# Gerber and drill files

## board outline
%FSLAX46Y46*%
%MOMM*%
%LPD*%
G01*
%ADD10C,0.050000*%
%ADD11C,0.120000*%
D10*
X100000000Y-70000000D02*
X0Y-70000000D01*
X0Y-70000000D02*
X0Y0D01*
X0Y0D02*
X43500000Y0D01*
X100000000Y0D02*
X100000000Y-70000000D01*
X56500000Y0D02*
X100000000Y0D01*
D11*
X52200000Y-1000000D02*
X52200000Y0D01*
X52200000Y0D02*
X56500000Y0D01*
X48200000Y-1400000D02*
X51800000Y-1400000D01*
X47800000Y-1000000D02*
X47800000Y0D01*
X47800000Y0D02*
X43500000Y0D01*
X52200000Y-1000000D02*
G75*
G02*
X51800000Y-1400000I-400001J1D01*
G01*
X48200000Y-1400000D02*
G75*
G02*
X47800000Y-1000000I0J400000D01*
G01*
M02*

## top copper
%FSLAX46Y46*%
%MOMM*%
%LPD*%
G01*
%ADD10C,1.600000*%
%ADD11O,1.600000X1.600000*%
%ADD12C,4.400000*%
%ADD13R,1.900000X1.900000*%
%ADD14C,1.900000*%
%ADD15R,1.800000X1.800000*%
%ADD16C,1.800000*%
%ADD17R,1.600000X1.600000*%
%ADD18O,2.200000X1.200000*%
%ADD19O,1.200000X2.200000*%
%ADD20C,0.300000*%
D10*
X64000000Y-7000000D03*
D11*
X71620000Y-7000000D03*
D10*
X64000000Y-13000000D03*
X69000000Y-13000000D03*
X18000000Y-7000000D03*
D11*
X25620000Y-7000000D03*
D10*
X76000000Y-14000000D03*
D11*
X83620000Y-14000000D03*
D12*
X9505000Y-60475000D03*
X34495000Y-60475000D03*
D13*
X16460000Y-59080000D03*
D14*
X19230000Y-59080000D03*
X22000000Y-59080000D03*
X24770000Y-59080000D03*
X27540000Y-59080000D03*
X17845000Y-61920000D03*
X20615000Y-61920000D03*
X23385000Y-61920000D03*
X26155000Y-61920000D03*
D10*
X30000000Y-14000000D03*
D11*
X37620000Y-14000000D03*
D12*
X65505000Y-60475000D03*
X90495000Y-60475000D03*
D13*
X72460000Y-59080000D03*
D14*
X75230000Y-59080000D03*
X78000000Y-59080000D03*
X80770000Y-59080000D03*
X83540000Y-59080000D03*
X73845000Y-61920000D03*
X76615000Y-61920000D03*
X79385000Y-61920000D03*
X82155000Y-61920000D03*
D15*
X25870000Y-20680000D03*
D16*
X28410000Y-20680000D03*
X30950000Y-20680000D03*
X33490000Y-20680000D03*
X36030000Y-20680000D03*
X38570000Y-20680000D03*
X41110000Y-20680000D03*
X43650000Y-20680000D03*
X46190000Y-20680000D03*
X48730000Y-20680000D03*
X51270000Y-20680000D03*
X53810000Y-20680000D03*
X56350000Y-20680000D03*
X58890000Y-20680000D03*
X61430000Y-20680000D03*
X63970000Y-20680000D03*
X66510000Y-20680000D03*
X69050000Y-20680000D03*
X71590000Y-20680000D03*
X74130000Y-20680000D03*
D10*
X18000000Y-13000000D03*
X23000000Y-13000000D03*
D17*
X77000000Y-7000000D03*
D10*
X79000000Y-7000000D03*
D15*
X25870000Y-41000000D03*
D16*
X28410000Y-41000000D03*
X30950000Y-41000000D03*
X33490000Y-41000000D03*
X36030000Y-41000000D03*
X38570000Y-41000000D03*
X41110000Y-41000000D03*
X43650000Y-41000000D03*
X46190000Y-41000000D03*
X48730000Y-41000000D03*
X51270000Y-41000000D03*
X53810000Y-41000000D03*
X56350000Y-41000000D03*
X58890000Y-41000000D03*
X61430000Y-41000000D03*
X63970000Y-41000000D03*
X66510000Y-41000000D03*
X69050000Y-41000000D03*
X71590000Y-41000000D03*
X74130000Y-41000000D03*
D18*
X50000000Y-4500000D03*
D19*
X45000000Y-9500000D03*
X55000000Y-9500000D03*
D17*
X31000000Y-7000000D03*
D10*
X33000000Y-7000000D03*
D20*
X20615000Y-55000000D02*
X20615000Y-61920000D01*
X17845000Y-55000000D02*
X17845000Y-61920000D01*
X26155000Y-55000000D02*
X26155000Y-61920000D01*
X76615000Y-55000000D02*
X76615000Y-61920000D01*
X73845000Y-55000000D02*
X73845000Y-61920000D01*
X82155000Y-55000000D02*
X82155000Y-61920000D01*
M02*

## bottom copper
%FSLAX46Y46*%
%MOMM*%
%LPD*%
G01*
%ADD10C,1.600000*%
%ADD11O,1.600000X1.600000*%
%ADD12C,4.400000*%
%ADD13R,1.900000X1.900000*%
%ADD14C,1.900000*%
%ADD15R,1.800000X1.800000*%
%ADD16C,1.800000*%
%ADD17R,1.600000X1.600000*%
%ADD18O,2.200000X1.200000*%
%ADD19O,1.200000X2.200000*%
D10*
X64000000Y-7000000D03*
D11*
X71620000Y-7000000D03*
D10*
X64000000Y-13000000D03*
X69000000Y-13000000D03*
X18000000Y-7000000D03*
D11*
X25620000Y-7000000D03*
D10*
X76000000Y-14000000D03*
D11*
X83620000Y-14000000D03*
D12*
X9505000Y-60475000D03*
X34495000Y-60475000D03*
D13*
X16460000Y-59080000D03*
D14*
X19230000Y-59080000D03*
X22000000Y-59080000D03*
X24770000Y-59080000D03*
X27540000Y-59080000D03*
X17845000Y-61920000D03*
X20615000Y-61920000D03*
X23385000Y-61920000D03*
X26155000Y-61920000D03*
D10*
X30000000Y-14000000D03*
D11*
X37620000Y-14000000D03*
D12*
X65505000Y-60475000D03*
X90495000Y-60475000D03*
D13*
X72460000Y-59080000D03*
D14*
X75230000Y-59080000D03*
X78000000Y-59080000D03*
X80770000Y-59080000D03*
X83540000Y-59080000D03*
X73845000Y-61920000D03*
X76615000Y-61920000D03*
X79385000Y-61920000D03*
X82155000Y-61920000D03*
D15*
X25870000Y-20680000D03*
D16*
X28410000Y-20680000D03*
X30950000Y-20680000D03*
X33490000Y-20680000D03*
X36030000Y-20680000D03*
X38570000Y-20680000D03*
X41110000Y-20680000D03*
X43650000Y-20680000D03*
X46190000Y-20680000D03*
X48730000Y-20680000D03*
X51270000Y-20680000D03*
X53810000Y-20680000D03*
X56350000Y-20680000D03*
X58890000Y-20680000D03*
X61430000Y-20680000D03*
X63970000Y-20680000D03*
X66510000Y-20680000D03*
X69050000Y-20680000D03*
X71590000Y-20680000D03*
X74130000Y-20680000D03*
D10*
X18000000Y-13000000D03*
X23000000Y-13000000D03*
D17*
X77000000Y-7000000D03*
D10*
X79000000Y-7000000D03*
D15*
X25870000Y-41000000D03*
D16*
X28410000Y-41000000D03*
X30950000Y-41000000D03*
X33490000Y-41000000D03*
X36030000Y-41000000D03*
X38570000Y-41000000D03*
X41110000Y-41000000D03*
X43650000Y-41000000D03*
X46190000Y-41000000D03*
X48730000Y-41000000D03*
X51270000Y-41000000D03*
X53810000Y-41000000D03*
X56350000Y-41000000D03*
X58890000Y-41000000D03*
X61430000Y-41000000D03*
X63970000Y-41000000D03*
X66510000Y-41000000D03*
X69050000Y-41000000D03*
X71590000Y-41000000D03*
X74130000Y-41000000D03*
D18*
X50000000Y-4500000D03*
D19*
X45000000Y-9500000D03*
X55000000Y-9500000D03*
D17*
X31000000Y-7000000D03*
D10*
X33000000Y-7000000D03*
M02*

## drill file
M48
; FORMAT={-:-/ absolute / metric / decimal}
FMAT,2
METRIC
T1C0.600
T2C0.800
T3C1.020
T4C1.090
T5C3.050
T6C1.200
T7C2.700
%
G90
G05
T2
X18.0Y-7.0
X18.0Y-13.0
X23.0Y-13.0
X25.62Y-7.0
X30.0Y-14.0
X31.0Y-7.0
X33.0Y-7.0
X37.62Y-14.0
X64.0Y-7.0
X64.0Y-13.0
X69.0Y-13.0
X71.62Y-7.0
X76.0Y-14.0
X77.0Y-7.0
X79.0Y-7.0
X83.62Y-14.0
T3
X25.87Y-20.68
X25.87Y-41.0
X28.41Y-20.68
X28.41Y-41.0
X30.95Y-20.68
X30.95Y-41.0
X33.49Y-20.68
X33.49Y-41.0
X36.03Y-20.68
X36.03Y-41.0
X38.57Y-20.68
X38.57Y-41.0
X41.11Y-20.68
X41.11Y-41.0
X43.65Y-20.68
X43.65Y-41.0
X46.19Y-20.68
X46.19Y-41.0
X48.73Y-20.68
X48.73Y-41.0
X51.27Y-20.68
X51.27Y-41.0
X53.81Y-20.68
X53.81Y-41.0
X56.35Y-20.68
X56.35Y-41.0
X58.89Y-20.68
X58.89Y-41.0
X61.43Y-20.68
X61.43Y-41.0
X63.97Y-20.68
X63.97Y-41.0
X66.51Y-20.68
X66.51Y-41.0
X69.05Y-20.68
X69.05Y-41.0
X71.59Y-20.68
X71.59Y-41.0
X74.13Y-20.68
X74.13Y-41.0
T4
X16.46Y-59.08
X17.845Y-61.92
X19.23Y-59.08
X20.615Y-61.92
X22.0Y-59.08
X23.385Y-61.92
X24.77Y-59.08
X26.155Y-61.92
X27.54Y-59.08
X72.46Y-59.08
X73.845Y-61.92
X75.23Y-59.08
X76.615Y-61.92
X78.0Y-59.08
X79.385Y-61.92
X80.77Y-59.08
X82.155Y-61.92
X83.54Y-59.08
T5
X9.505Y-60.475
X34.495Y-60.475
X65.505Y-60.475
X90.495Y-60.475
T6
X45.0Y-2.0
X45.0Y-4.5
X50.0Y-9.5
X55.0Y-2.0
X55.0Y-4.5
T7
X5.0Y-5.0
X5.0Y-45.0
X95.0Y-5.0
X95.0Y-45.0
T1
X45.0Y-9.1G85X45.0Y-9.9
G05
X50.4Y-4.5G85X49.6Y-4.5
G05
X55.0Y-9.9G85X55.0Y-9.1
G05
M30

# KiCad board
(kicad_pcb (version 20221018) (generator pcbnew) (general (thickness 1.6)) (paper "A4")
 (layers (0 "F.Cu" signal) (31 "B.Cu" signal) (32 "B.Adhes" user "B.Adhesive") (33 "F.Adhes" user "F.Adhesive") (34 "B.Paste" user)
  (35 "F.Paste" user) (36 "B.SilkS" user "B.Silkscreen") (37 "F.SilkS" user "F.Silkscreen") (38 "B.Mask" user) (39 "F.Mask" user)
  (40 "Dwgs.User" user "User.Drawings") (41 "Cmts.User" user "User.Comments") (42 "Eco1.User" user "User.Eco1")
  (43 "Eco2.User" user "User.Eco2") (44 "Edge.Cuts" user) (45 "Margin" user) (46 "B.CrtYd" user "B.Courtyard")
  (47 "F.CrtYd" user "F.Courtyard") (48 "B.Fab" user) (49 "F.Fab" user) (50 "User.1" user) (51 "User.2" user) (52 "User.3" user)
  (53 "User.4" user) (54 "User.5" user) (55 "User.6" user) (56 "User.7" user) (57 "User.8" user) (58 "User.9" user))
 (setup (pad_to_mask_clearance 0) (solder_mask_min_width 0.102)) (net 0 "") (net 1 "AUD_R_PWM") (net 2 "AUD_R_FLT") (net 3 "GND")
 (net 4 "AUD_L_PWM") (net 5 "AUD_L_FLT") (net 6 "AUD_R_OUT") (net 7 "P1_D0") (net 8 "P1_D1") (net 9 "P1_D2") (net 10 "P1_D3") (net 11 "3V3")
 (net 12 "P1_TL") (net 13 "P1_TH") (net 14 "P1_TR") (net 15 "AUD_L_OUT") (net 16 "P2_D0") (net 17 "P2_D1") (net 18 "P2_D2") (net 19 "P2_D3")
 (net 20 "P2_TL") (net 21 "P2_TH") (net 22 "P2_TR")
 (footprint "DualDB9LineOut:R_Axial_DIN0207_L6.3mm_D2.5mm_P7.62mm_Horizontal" (layer "F.Cu") (at 64 7)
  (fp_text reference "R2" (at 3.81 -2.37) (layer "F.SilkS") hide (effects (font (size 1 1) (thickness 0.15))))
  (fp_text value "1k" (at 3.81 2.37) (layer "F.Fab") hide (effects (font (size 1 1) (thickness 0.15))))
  (pad "1" thru_hole circle (at 0 0) (size 1.6 1.6) (drill 0.8) (layers "*.Cu" "*.Mask") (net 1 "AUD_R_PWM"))
  (pad "2" thru_hole oval (at 7.62 0) (size 1.6 1.6) (drill 0.8) (layers "*.Cu" "*.Mask") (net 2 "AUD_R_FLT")))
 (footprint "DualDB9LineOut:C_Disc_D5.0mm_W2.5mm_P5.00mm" (layer "F.Cu") (at 64 13)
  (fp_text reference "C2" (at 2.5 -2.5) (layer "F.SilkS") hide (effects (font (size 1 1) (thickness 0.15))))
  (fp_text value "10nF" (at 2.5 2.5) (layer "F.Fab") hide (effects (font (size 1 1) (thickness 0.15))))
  (pad "1" thru_hole circle (at 0 0) (size 1.6 1.6) (drill 0.8) (layers "*.Cu" "*.Mask") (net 2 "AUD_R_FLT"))
  (pad "2" thru_hole circle (at 5 0) (size 1.6 1.6) (drill 0.8) (layers "*.Cu" "*.Mask") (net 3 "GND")))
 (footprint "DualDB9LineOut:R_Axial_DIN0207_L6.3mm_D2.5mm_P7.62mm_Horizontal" (layer "F.Cu") (at 18 7)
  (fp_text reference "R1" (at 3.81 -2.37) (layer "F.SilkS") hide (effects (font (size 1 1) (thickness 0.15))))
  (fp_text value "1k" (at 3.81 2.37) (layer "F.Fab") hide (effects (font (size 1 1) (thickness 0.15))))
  (pad "1" thru_hole circle (at 0 0) (size 1.6 1.6) (drill 0.8) (layers "*.Cu" "*.Mask") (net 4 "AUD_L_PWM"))
  (pad "2" thru_hole oval (at 7.62 0) (size 1.6 1.6) (drill 0.8) (layers "*.Cu" "*.Mask") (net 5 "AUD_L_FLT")))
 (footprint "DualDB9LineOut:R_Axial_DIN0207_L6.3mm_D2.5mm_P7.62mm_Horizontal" (layer "F.Cu") (at 76 14)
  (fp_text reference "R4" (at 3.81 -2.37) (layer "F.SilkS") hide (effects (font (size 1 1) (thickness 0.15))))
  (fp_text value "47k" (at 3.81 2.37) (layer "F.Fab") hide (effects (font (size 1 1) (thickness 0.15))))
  (pad "1" thru_hole circle (at 0 0) (size 1.6 1.6) (drill 0.8) (layers "*.Cu" "*.Mask") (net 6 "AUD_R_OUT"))
  (pad "2" thru_hole oval (at 7.62 0) (size 1.6 1.6) (drill 0.8) (layers "*.Cu" "*.Mask") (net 3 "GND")))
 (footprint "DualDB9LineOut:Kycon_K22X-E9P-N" (layer "F.Cu") (at 16.46 59.08)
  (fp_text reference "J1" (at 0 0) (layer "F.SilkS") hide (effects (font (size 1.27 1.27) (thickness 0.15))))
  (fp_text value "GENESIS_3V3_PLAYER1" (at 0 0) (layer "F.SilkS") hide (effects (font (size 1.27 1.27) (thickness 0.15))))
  (pad "0" thru_hole circle (at -6.955 1.395) (size 4.4 4.4) (drill 3.05) (layers "F&B.Cu" "*.Mask") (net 3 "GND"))
  (pad "0" thru_hole circle (at 18.035 1.395) (size 4.4 4.4) (drill 3.05) (layers "F&B.Cu" "*.Mask") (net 3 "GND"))
  (pad "1" thru_hole rect (at 0 0) (size 1.9 1.9) (drill 1.09) (layers "F&B.Cu" "*.Mask") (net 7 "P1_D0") (thermal_bridge_angle 45))
  (pad "2" thru_hole circle (at 2.77 0) (size 1.9 1.9) (drill 1.09) (layers "F&B.Cu" "*.Mask") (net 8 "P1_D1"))
  (pad "3" thru_hole circle (at 5.54 0) (size 1.9 1.9) (drill 1.09) (layers "F&B.Cu" "*.Mask") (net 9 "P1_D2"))
  (pad "4" thru_hole circle (at 8.31 0) (size 1.9 1.9) (drill 1.09) (layers "F&B.Cu" "*.Mask") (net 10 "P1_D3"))
  (pad "5" thru_hole circle (at 11.08 0) (size 1.9 1.9) (drill 1.09) (layers "F&B.Cu" "*.Mask") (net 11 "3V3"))
  (pad "6" thru_hole circle (at 1.385 2.84) (size 1.9 1.9) (drill 1.09) (layers "F&B.Cu" "*.Mask") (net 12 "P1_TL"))
  (pad "7" thru_hole circle (at 4.155 2.84) (size 1.9 1.9) (drill 1.09) (layers "F&B.Cu" "*.Mask") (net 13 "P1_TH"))
  (pad "8" thru_hole circle (at 6.925 2.84) (size 1.9 1.9) (drill 1.09) (layers "F&B.Cu" "*.Mask") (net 3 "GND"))
  (pad "9" thru_hole circle (at 9.695 2.84) (size 1.9 1.9) (drill 1.09) (layers "F&B.Cu" "*.Mask") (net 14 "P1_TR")))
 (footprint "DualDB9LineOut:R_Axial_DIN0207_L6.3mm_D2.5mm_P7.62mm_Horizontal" (layer "F.Cu") (at 30 14)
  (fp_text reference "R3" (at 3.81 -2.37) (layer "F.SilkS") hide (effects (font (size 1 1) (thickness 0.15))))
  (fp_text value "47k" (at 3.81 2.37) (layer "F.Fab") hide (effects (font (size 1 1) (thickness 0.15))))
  (pad "1" thru_hole circle (at 0 0) (size 1.6 1.6) (drill 0.8) (layers "*.Cu" "*.Mask") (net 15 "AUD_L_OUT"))
  (pad "2" thru_hole oval (at 7.62 0) (size 1.6 1.6) (drill 0.8) (layers "*.Cu" "*.Mask") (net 3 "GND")))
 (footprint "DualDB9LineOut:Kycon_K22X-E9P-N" (layer "F.Cu") (at 72.46 59.08)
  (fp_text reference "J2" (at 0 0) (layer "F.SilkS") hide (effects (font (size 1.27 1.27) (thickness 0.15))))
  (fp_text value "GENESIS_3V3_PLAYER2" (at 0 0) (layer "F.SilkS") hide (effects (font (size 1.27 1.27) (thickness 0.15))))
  (pad "0" thru_hole circle (at -6.955 1.395) (size 4.4 4.4) (drill 3.05) (layers "F&B.Cu" "*.Mask") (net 3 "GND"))
  (pad "0" thru_hole circle (at 18.035 1.395) (size 4.4 4.4) (drill 3.05) (layers "F&B.Cu" "*.Mask") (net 3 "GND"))
  (pad "1" thru_hole rect (at 0 0) (size 1.9 1.9) (drill 1.09) (layers "F&B.Cu" "*.Mask") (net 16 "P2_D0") (thermal_bridge_angle 45))
  (pad "2" thru_hole circle (at 2.77 0) (size 1.9 1.9) (drill 1.09) (layers "F&B.Cu" "*.Mask") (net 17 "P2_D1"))
  (pad "3" thru_hole circle (at 5.54 0) (size 1.9 1.9) (drill 1.09) (layers "F&B.Cu" "*.Mask") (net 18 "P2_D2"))
  (pad "4" thru_hole circle (at 8.31 0) (size 1.9 1.9) (drill 1.09) (layers "F&B.Cu" "*.Mask") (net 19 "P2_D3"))
  (pad "5" thru_hole circle (at 11.08 0) (size 1.9 1.9) (drill 1.09) (layers "F&B.Cu" "*.Mask") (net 11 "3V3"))
  (pad "6" thru_hole circle (at 1.385 2.84) (size 1.9 1.9) (drill 1.09) (layers "F&B.Cu" "*.Mask") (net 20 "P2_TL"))
  (pad "7" thru_hole circle (at 4.155 2.84) (size 1.9 1.9) (drill 1.09) (layers "F&B.Cu" "*.Mask") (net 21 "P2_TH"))
  (pad "8" thru_hole circle (at 6.925 2.84) (size 1.9 1.9) (drill 1.09) (layers "F&B.Cu" "*.Mask") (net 3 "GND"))
  (pad "9" thru_hole circle (at 9.695 2.84) (size 1.9 1.9) (drill 1.09) (layers "F&B.Cu" "*.Mask") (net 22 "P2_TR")))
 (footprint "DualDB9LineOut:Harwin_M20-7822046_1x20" (layer "F.Cu") (at 25.87 20.68 90)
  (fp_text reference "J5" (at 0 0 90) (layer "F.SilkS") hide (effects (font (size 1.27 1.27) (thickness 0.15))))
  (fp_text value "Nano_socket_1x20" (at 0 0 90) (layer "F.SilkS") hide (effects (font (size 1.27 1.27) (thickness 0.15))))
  (pad "1" thru_hole rect (at 0 0 90) (size 1.8 1.8) (drill 1.02) (layers "F&B.Cu" "*.Mask") (thermal_bridge_angle 45))
  (pad "2" thru_hole circle (at 0 2.54 90) (size 1.8 1.8) (drill 1.02) (layers "F&B.Cu" "*.Mask"))
  (pad "3" thru_hole circle (at 0 5.08 90) (size 1.8 1.8) (drill 1.02) (layers "F&B.Cu" "*.Mask"))
  (pad "4" thru_hole circle (at 0 7.62 90) (size 1.8 1.8) (drill 1.02) (layers "F&B.Cu" "*.Mask"))
  (pad "5" thru_hole circle (at 0 10.16 90) (size 1.8 1.8) (drill 1.02) (layers "F&B.Cu" "*.Mask") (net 16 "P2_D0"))
  (pad "6" thru_hole circle (at 0 12.7 90) (size 1.8 1.8) (drill 1.02) (layers "F&B.Cu" "*.Mask") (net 17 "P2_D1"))
  (pad "7" thru_hole circle (at 0 15.24 90) (size 1.8 1.8) (drill 1.02) (layers "F&B.Cu" "*.Mask"))
  (pad "8" thru_hole circle (at 0 17.78 90) (size 1.8 1.8) (drill 1.02) (layers "F&B.Cu" "*.Mask"))
  (pad "9" thru_hole circle (at 0 20.32 90) (size 1.8 1.8) (drill 1.02) (layers "F&B.Cu" "*.Mask") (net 18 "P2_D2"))
  (pad "10" thru_hole circle (at 0 22.86 90) (size 1.8 1.8) (drill 1.02) (layers "F&B.Cu" "*.Mask") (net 19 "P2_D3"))
  (pad "11" thru_hole circle (at 0 25.4 90) (size 1.8 1.8) (drill 1.02) (layers "F&B.Cu" "*.Mask"))
  (pad "12" thru_hole circle (at 0 27.94 90) (size 1.8 1.8) (drill 1.02) (layers "F&B.Cu" "*.Mask") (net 20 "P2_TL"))
  (pad "13" thru_hole circle (at 0 30.48 90) (size 1.8 1.8) (drill 1.02) (layers "F&B.Cu" "*.Mask"))
  (pad "14" thru_hole circle (at 0 33.02 90) (size 1.8 1.8) (drill 1.02) (layers "F&B.Cu" "*.Mask"))
  (pad "15" thru_hole circle (at 0 35.56 90) (size 1.8 1.8) (drill 1.02) (layers "F&B.Cu" "*.Mask") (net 3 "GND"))
  (pad "16" thru_hole circle (at 0 38.1 90) (size 1.8 1.8) (drill 1.02) (layers "F&B.Cu" "*.Mask") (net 11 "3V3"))
  (pad "17" thru_hole circle (at 0 40.64 90) (size 1.8 1.8) (drill 1.02) (layers "F&B.Cu" "*.Mask") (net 21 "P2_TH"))
  (pad "18" thru_hole circle (at 0 43.18 90) (size 1.8 1.8) (drill 1.02) (layers "F&B.Cu" "*.Mask") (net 22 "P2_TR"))
  (pad "19" thru_hole circle (at 0 45.72 90) (size 1.8 1.8) (drill 1.02) (layers "F&B.Cu" "*.Mask"))
  (pad "20" thru_hole circle (at 0 48.26 90) (size 1.8 1.8) (drill 1.02) (layers "F&B.Cu" "*.Mask")))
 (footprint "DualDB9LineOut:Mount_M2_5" (layer "F.Cu") (at 5 5)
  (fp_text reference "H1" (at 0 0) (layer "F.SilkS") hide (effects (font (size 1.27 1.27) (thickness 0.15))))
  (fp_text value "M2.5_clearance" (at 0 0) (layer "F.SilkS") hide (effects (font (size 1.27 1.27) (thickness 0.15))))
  (pad "" np_thru_hole circle (at 0 0) (size 2.7 2.7) (drill 2.7) (layers "F&B.Cu" "*.Mask")))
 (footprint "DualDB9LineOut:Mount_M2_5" (layer "F.Cu") (at 5 45)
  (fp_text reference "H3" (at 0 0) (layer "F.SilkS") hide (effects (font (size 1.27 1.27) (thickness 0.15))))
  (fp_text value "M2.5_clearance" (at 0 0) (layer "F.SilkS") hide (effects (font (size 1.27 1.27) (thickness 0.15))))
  (pad "" np_thru_hole circle (at 0 0) (size 2.7 2.7) (drill 2.7) (layers "F&B.Cu" "*.Mask")))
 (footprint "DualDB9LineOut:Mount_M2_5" (layer "F.Cu") (at 95 5)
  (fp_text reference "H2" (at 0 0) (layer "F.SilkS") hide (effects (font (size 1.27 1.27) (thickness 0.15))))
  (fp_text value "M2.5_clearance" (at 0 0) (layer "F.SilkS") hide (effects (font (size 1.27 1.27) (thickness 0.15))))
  (pad "" np_thru_hole circle (at 0 0) (size 2.7 2.7) (drill 2.7) (layers "F&B.Cu" "*.Mask")))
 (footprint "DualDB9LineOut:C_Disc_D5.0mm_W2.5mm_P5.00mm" (layer "F.Cu") (at 18 13)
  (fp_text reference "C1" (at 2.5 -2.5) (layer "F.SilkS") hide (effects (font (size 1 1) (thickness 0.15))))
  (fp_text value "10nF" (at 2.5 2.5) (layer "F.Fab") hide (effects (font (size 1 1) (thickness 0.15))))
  (pad "1" thru_hole circle (at 0 0) (size 1.6 1.6) (drill 0.8) (layers "*.Cu" "*.Mask") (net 5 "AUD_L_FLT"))
  (pad "2" thru_hole circle (at 5 0) (size 1.6 1.6) (drill 0.8) (layers "*.Cu" "*.Mask") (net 3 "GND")))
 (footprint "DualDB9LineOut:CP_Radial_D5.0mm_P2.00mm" (layer "F.Cu") (at 77 7)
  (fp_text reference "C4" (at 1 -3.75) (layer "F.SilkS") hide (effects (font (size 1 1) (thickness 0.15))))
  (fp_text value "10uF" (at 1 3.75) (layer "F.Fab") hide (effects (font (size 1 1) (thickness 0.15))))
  (pad "1" thru_hole rect (at 0 0) (size 1.6 1.6) (drill 0.8) (layers "*.Cu" "*.Mask") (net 2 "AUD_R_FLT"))
  (pad "2" thru_hole circle (at 2 0) (size 1.6 1.6) (drill 0.8) (layers "*.Cu" "*.Mask") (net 6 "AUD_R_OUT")))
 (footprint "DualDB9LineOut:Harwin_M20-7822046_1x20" (layer "F.Cu") (at 25.87 41 90)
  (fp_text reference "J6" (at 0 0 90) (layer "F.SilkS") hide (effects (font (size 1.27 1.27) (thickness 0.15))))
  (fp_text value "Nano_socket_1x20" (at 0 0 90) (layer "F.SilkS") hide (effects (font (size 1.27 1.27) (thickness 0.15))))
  (pad "1" thru_hole rect (at 0 0 90) (size 1.8 1.8) (drill 1.02) (layers "F&B.Cu" "*.Mask") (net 7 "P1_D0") (thermal_bridge_angle 45))
  (pad "2" thru_hole circle (at 0 2.54 90) (size 1.8 1.8) (drill 1.02) (layers "F&B.Cu" "*.Mask") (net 8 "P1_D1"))
  (pad "3" thru_hole circle (at 0 5.08 90) (size 1.8 1.8) (drill 1.02) (layers "F&B.Cu" "*.Mask"))
  (pad "4" thru_hole circle (at 0 7.62 90) (size 1.8 1.8) (drill 1.02) (layers "F&B.Cu" "*.Mask"))
  (pad "5" thru_hole circle (at 0 10.16 90) (size 1.8 1.8) (drill 1.02) (layers "F&B.Cu" "*.Mask") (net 9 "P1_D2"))
  (pad "6" thru_hole circle (at 0 12.7 90) (size 1.8 1.8) (drill 1.02) (layers "F&B.Cu" "*.Mask"))
  (pad "7" thru_hole circle (at 0 15.24 90) (size 1.8 1.8) (drill 1.02) (layers "F&B.Cu" "*.Mask"))
  (pad "8" thru_hole circle (at 0 17.78 90) (size 1.8 1.8) (drill 1.02) (layers "F&B.Cu" "*.Mask") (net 10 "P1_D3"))
  (pad "9" thru_hole circle (at 0 20.32 90) (size 1.8 1.8) (drill 1.02) (layers "F&B.Cu" "*.Mask") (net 12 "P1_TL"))
  (pad "10" thru_hole circle (at 0 22.86 90) (size 1.8 1.8) (drill 1.02) (layers "F&B.Cu" "*.Mask"))
  (pad "11" thru_hole circle (at 0 25.4 90) (size 1.8 1.8) (drill 1.02) (layers "F&B.Cu" "*.Mask"))
  (pad "12" thru_hole circle (at 0 27.94 90) (size 1.8 1.8) (drill 1.02) (layers "F&B.Cu" "*.Mask") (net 13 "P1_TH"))
  (pad "13" thru_hole circle (at 0 30.48 90) (size 1.8 1.8) (drill 1.02) (layers "F&B.Cu" "*.Mask") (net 14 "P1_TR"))
  (pad "14" thru_hole circle (at 0 33.02 90) (size 1.8 1.8) (drill 1.02) (layers "F&B.Cu" "*.Mask") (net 4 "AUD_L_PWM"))
  (pad "15" thru_hole circle (at 0 35.56 90) (size 1.8 1.8) (drill 1.02) (layers "F&B.Cu" "*.Mask") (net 1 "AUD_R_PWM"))
  (pad "16" thru_hole circle (at 0 38.1 90) (size 1.8 1.8) (drill 1.02) (layers "F&B.Cu" "*.Mask"))
  (pad "17" thru_hole circle (at 0 40.64 90) (size 1.8 1.8) (drill 1.02) (layers "F&B.Cu" "*.Mask"))
  (pad "18" thru_hole circle (at 0 43.18 90) (size 1.8 1.8) (drill 1.02) (layers "F&B.Cu" "*.Mask"))
  (pad "19" thru_hole circle (at 0 45.72 90) (size 1.8 1.8) (drill 1.02) (layers "F&B.Cu" "*.Mask") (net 11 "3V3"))
  (pad "20" thru_hole circle (at 0 48.26 90) (size 1.8 1.8) (drill 1.02) (layers "F&B.Cu" "*.Mask") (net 3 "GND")))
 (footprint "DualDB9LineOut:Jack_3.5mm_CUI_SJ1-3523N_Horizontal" (layer "F.Cu") (at 50 4.5 180)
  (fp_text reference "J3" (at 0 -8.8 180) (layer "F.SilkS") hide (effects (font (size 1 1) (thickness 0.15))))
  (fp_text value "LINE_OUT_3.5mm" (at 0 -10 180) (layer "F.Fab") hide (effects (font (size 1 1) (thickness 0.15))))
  (fp_line (start -2.2 3.5) (end -2.2 4.5) (stroke (width 0.12) (type solid)) (layer "Edge.Cuts"))
  (fp_line (start -2.2 4.5) (end -6.5 4.5) (stroke (width 0.12) (type solid)) (layer "Edge.Cuts"))
  (fp_line (start 1.8 3.1) (end -1.8 3.1) (stroke (width 0.12) (type solid)) (layer "Edge.Cuts"))
  (fp_line (start 2.2 3.5) (end 2.2 4.5) (stroke (width 0.12) (type solid)) (layer "Edge.Cuts"))
  (fp_line (start 2.2 4.5) (end 6.5 4.5) (stroke (width 0.12) (type solid)) (layer "Edge.Cuts"))
  (fp_arc (start -2.2 3.5) (mid -2.082843 3.217158) (end -1.8 3.1) (stroke (width 0.12) (type solid)) (layer "Edge.Cuts"))
  (fp_arc (start 1.8 3.1) (mid 2.082843 3.217157) (end 2.2 3.5) (stroke (width 0.12) (type solid)) (layer "Edge.Cuts"))
  (pad "" np_thru_hole circle (at -5 0 180) (size 1.2 1.2) (drill 1.2) (layers "F&B.Cu" "*.Mask"))
  (pad "" np_thru_hole circle (at -5 2.5 180) (size 1.2 1.2) (drill 1.2) (layers "F&B.Cu" "*.Mask"))
  (pad "" np_thru_hole circle (at 0 -5 180) (size 1.2 1.2) (drill 1.2) (layers "F&B.Cu" "*.Mask"))
  (pad "" np_thru_hole circle (at 5 0 180) (size 1.2 1.2) (drill 1.2) (layers "F&B.Cu" "*.Mask"))
  (pad "" np_thru_hole circle (at 5 2.5 180) (size 1.2 1.2) (drill 1.2) (layers "F&B.Cu" "*.Mask"))
  (pad "1" thru_hole oval (at 0 0 180) (size 2.2 1.2) (drill oval 1.4 0.6) (layers "*.Cu" "*.Mask") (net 3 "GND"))
  (pad "2" thru_hole oval (at 5 -5) (size 1.2 2.2) (drill oval 0.6 1.4) (layers "*.Cu" "*.Mask") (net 15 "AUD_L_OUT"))
  (pad "3" thru_hole oval (at -5 -5 180) (size 1.2 2.2) (drill oval 0.6 1.4) (layers "*.Cu" "*.Mask") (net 6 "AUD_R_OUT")))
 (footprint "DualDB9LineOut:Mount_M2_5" (layer "F.Cu") (at 95 45)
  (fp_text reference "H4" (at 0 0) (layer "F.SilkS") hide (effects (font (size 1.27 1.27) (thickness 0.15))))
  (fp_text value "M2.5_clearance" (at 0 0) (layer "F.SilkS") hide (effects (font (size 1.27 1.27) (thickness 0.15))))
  (pad "" np_thru_hole circle (at 0 0) (size 2.7 2.7) (drill 2.7) (layers "F&B.Cu" "*.Mask")))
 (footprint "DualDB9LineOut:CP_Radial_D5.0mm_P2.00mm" (layer "F.Cu") (at 31 7)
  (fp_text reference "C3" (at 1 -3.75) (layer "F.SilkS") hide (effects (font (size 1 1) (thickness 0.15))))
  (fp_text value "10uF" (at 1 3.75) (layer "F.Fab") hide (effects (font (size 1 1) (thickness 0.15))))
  (pad "1" thru_hole rect (at 0 0) (size 1.6 1.6) (drill 0.8) (layers "*.Cu" "*.Mask") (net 5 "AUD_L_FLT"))
  (pad "2" thru_hole circle (at 2 0) (size 1.6 1.6) (drill 0.8) (layers "*.Cu" "*.Mask") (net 15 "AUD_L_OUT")))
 (gr_line (start 100 70) (end 0 70) (stroke (width 0.05) (type default)) (layer "Edge.Cuts"))
 (gr_line (start 0 70) (end 0 0) (stroke (width 0.05) (type default)) (layer "Edge.Cuts"))
 (gr_line (start 0 0) (end 43.5 0) (stroke (width 0.05) (type default)) (layer "Edge.Cuts"))
 (gr_line (start 100 0) (end 100 70) (stroke (width 0.05) (type default)) (layer "Edge.Cuts"))
 (gr_line (start 56.5 0) (end 100 0) (stroke (width 0.05) (type default)) (layer "Edge.Cuts"))
 (segment (start 20.615 55) (end 20.615 61.92) (width 0.3) (layer "F.Cu") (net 13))
 (segment (start 17.845 55) (end 17.845 61.92) (width 0.3) (layer "F.Cu") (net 12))
 (segment (start 26.155 55) (end 26.155 61.92) (width 0.3) (layer "F.Cu") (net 14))
 (segment (start 76.615 55) (end 76.615 61.92) (width 0.3) (layer "F.Cu") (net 21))
 (segment (start 73.845 55) (end 73.845 61.92) (width 0.3) (layer "F.Cu") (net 20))
 (segment (start 82.155 55) (end 82.155 61.92) (width 0.3) (layer "F.Cu") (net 22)))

